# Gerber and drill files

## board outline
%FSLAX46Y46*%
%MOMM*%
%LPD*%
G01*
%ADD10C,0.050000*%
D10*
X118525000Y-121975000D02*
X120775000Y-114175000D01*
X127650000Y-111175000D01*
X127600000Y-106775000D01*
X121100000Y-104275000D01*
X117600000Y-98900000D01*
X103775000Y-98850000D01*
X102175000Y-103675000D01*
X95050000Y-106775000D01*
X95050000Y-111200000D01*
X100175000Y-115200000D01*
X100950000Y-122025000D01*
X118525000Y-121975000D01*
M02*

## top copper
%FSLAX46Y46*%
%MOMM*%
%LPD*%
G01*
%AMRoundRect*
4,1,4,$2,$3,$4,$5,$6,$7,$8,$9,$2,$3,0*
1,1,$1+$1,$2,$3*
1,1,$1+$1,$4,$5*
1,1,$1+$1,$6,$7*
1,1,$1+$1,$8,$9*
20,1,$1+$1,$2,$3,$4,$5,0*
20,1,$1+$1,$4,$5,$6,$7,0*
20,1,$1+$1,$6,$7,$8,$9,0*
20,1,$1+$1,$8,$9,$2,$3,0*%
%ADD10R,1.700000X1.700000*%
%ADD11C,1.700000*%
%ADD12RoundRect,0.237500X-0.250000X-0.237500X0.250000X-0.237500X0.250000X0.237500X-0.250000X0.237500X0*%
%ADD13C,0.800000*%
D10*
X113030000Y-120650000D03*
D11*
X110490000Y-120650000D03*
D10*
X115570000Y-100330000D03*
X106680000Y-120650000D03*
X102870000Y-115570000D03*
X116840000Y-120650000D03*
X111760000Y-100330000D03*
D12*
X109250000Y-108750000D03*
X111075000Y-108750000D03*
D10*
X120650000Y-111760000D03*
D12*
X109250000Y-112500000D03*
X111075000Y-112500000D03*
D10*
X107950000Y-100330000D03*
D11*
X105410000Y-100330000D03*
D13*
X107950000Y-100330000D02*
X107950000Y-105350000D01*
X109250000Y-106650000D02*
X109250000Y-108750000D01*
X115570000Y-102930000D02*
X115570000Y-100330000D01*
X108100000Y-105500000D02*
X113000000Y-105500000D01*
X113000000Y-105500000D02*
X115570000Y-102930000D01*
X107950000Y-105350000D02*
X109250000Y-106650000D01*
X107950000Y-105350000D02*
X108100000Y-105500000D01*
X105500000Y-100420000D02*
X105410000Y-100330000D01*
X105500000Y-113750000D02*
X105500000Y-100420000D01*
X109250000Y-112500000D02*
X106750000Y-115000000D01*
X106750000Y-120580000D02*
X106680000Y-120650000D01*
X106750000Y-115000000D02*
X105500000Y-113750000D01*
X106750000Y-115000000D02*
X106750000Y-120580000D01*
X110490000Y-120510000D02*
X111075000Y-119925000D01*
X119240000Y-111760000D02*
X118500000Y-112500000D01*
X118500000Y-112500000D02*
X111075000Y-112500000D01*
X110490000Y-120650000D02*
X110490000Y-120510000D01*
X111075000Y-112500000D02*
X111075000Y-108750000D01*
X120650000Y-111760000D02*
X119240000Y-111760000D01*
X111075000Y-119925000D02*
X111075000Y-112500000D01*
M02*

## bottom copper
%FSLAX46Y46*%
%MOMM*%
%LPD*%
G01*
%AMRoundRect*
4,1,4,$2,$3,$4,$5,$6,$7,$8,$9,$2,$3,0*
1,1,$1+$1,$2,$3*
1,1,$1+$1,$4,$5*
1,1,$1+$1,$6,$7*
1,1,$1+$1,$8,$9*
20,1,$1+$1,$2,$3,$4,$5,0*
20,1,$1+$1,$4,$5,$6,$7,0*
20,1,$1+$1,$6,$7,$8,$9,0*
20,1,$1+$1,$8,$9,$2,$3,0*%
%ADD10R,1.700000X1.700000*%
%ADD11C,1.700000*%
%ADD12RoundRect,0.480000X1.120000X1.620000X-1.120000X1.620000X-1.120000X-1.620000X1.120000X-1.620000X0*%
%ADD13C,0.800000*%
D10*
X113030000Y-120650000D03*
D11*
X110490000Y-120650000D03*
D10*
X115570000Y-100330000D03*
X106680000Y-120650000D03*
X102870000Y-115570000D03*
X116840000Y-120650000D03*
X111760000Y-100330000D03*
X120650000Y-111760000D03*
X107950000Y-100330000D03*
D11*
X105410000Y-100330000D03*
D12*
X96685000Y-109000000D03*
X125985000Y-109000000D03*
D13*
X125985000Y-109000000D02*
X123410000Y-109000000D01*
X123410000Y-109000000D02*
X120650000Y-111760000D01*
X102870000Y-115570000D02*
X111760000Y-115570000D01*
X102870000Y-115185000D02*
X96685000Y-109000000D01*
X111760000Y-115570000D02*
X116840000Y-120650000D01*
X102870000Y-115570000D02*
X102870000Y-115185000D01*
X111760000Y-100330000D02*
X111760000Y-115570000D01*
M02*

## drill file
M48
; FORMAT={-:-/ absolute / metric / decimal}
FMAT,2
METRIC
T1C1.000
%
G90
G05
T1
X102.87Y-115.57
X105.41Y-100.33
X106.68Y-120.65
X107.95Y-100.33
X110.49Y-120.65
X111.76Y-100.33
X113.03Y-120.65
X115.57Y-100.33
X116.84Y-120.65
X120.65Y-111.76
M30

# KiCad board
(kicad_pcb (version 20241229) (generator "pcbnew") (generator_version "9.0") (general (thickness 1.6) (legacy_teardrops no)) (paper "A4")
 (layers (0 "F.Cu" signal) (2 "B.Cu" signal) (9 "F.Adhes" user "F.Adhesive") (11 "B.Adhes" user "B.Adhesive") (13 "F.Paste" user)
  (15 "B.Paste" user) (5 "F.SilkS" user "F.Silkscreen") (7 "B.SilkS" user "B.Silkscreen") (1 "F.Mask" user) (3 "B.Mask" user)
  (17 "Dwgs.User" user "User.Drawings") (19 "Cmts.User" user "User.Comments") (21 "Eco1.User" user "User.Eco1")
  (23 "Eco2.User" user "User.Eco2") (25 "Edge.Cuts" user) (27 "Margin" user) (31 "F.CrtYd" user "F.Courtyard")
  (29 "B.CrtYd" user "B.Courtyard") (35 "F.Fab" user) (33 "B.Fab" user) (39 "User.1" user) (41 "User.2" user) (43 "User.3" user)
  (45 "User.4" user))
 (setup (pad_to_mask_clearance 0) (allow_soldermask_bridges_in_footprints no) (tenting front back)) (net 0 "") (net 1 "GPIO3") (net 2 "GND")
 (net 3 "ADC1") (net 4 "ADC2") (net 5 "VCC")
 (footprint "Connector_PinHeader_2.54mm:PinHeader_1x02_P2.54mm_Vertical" (layer "F.Cu") (at 113.03 120.65 -90)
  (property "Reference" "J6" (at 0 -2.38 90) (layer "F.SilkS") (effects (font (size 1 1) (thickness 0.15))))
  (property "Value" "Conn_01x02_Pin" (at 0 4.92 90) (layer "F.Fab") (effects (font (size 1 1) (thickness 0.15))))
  (pad "1" thru_hole rect (at 0 0 270) (size 1.7 1.7) (drill 1) (layers "*.Cu" "*.Mask") (remove_unused_layers no) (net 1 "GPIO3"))
  (pad "2" thru_hole circle (at 0 2.54 270) (size 1.7 1.7) (drill 1) (layers "*.Cu" "*.Mask") (remove_unused_layers no) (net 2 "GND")))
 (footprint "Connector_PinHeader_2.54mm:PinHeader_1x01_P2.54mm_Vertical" (layer "F.Cu") (at 115.57 100.33)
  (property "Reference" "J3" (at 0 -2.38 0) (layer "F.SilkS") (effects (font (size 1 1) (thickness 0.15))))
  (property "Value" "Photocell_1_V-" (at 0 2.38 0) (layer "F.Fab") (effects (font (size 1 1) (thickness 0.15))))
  (pad "1" thru_hole rect (at 0 0) (size 1.7 1.7) (drill 1) (layers "*.Cu" "*.Mask") (remove_unused_layers no) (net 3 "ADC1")))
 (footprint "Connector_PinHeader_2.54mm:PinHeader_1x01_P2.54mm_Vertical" (layer "F.Cu") (at 106.68 120.65)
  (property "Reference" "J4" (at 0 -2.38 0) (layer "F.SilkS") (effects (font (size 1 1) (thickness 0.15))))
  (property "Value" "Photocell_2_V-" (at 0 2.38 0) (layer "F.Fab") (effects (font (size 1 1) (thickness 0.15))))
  (pad "1" thru_hole rect (at 0 0) (size 1.7 1.7) (drill 1) (layers "*.Cu" "*.Mask") (remove_unused_layers no) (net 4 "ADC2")))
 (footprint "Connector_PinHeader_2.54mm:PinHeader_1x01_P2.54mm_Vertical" (layer "F.Cu") (at 102.87 115.57)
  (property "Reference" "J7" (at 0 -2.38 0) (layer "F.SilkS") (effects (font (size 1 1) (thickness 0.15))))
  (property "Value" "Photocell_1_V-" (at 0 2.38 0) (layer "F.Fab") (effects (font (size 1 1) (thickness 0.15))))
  (pad "1" thru_hole rect (at 0 0) (size 1.7 1.7) (drill 1) (layers "*.Cu" "*.Mask") (remove_unused_layers no) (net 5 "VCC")))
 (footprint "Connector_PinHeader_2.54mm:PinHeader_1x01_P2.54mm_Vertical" (layer "F.Cu") (at 116.84 120.65)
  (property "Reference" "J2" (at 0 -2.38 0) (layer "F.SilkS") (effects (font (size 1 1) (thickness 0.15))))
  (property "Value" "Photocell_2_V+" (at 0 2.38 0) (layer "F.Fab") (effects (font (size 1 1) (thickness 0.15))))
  (pad "1" thru_hole rect (at 0 0) (size 1.7 1.7) (drill 1) (layers "*.Cu" "*.Mask") (remove_unused_layers no) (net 5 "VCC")))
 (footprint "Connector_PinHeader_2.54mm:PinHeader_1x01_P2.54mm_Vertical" (layer "F.Cu") (at 111.76 100.33)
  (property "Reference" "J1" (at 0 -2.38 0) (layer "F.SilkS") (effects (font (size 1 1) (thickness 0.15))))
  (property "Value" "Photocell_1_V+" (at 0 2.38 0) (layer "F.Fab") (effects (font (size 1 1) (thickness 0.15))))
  (pad "1" thru_hole rect (at 0 0) (size 1.7 1.7) (drill 1) (layers "*.Cu" "*.Mask") (remove_unused_layers no) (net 5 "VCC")))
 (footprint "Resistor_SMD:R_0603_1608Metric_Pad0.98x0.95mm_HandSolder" (layer "F.Cu") (at 110.1625 108.75)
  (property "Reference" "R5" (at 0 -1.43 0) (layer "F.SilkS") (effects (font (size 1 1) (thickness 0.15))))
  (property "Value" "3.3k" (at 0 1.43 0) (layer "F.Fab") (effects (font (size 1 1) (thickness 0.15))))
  (pad "1" smd roundrect (at -0.9125 0) (size 0.975 0.95) (layers "F.Cu" "F.Mask" "F.Paste") (roundrect_rratio 0.25) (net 3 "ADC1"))
  (pad "2" smd roundrect (at 0.9125 0) (size 0.975 0.95) (layers "F.Cu" "F.Mask" "F.Paste") (roundrect_rratio 0.25) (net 2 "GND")))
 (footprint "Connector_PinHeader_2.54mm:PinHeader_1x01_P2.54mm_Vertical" (layer "F.Cu") (at 120.65 111.76)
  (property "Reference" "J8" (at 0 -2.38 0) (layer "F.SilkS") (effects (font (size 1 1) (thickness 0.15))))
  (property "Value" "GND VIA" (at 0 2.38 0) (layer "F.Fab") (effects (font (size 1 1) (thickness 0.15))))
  (pad "1" thru_hole rect (at 0 0) (size 1.7 1.7) (drill 1) (layers "*.Cu" "*.Mask") (remove_unused_layers no) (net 2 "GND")))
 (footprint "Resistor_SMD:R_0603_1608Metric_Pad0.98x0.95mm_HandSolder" (layer "F.Cu") (at 110.1625 112.5)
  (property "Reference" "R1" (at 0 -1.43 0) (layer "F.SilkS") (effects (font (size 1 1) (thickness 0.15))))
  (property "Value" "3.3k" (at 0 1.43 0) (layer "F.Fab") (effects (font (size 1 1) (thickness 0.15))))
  (pad "1" smd roundrect (at -0.9125 0) (size 0.975 0.95) (layers "F.Cu" "F.Mask" "F.Paste") (roundrect_rratio 0.25) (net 4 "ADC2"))
  (pad "2" smd roundrect (at 0.9125 0) (size 0.975 0.95) (layers "F.Cu" "F.Mask" "F.Paste") (roundrect_rratio 0.25) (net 2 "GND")))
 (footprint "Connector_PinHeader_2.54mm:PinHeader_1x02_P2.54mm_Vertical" (layer "F.Cu") (at 107.95 100.33 -90)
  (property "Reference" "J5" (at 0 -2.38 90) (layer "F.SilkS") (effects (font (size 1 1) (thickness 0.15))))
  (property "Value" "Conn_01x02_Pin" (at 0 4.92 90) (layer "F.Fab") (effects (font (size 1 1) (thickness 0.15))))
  (pad "1" thru_hole rect (at 0 0 270) (size 1.7 1.7) (drill 1) (layers "*.Cu" "*.Mask") (remove_unused_layers no) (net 3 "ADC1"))
  (pad "2" thru_hole circle (at 0 2.54 270) (size 1.7 1.7) (drill 1) (layers "*.Cu" "*.Mask") (remove_unused_layers no) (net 4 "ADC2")))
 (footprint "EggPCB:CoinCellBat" (layer "B.Cu") (at 111.335 109 180)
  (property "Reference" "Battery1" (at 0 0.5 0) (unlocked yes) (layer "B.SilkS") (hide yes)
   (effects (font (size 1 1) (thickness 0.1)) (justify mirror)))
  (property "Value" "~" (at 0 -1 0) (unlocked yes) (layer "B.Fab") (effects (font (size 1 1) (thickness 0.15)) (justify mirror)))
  (pad "1" smd roundrect (at 14.65 0 180) (size 3.2 4.2) (layers "B.Cu" "B.Mask" "B.Paste") (roundrect_rratio 0.15) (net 5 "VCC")
   (thermal_bridge_angle 45))
  (pad "2" smd roundrect (at -14.65 0 180) (size 3.2 4.2) (layers "B.Cu" "B.Mask" "B.Paste") (roundrect_rratio 0.15) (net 2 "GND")
   (thermal_bridge_angle 45)))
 (gr_poly
  (pts (xy 118.525 121.975) (xy 120.775 114.175) (xy 127.65 111.175) (xy 127.6 106.775) (xy 121.1 104.275) (xy 117.6 98.9)
   (xy 103.775 98.85) (xy 102.175 103.675) (xy 95.05 106.775) (xy 95.05 111.2) (xy 100.175 115.2) (xy 100.95 122.025))
  (stroke (width 0.05) (type solid)) (fill no) (layer "Edge.Cuts"))
 (segment (start 107.95 100.33) (end 107.95 105.35) (width 0.8) (layer "F.Cu") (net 3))
 (segment (start 109.25 106.65) (end 109.25 108.75) (width 0.8) (layer "F.Cu") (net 3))
 (segment (start 115.57 102.93) (end 115.57 100.33) (width 0.8) (layer "F.Cu") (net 3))
 (segment (start 108.1 105.5) (end 113 105.5) (width 0.8) (layer "F.Cu") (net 3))
 (segment (start 113 105.5) (end 115.57 102.93) (width 0.8) (layer "F.Cu") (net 3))
 (segment (start 107.95 105.35) (end 109.25 106.65) (width 0.8) (layer "F.Cu") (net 3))
 (segment (start 107.95 105.35) (end 108.1 105.5) (width 0.8) (layer "F.Cu") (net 3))
 (segment (start 105.5 100.42) (end 105.41 100.33) (width 0.8) (layer "F.Cu") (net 4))
 (segment (start 105.5 113.75) (end 105.5 100.42) (width 0.8) (layer "F.Cu") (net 4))
 (segment (start 109.25 112.5) (end 106.75 115) (width 0.8) (layer "F.Cu") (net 4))
 (segment (start 106.75 120.58) (end 106.68 120.65) (width 0.8) (layer "F.Cu") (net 4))
 (segment (start 106.75 115) (end 105.5 113.75) (width 0.8) (layer "F.Cu") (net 4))
 (segment (start 106.75 115) (end 106.75 120.58) (width 0.8) (layer "F.Cu") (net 4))
 (segment (start 110.49 120.51) (end 111.075 119.925) (width 0.8) (layer "F.Cu") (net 2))
 (segment (start 119.24 111.76) (end 118.5 112.5) (width 0.8) (layer "F.Cu") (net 2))
 (segment (start 118.5 112.5) (end 111.075 112.5) (width 0.8) (layer "F.Cu") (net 2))
 (segment (start 110.49 120.65) (end 110.49 120.51) (width 0.8) (layer "F.Cu") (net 2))
 (segment (start 111.075 112.5) (end 111.075 108.75) (width 0.8) (layer "F.Cu") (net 2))
 (segment (start 120.65 111.76) (end 119.24 111.76) (width 0.8) (layer "F.Cu") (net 2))
 (segment (start 111.075 119.925) (end 111.075 112.5) (width 0.8) (layer "F.Cu") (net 2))
 (segment (start 125.985 109) (end 123.41 109) (width 0.8) (layer "B.Cu") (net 2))
 (segment (start 123.41 109) (end 120.65 111.76) (width 0.8) (layer "B.Cu") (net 2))
 (segment (start 102.87 115.57) (end 111.76 115.57) (width 0.8) (layer "B.Cu") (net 5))
 (segment (start 102.87 115.185) (end 96.685 109) (width 0.8) (layer "B.Cu") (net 5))
 (segment (start 111.76 115.57) (end 116.84 120.65) (width 0.8) (layer "B.Cu") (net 5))
 (segment (start 102.87 115.57) (end 102.87 115.185) (width 0.8) (layer "B.Cu") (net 5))
 (segment (start 111.76 100.33) (end 111.76 115.57) (width 0.8) (layer "B.Cu") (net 5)))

